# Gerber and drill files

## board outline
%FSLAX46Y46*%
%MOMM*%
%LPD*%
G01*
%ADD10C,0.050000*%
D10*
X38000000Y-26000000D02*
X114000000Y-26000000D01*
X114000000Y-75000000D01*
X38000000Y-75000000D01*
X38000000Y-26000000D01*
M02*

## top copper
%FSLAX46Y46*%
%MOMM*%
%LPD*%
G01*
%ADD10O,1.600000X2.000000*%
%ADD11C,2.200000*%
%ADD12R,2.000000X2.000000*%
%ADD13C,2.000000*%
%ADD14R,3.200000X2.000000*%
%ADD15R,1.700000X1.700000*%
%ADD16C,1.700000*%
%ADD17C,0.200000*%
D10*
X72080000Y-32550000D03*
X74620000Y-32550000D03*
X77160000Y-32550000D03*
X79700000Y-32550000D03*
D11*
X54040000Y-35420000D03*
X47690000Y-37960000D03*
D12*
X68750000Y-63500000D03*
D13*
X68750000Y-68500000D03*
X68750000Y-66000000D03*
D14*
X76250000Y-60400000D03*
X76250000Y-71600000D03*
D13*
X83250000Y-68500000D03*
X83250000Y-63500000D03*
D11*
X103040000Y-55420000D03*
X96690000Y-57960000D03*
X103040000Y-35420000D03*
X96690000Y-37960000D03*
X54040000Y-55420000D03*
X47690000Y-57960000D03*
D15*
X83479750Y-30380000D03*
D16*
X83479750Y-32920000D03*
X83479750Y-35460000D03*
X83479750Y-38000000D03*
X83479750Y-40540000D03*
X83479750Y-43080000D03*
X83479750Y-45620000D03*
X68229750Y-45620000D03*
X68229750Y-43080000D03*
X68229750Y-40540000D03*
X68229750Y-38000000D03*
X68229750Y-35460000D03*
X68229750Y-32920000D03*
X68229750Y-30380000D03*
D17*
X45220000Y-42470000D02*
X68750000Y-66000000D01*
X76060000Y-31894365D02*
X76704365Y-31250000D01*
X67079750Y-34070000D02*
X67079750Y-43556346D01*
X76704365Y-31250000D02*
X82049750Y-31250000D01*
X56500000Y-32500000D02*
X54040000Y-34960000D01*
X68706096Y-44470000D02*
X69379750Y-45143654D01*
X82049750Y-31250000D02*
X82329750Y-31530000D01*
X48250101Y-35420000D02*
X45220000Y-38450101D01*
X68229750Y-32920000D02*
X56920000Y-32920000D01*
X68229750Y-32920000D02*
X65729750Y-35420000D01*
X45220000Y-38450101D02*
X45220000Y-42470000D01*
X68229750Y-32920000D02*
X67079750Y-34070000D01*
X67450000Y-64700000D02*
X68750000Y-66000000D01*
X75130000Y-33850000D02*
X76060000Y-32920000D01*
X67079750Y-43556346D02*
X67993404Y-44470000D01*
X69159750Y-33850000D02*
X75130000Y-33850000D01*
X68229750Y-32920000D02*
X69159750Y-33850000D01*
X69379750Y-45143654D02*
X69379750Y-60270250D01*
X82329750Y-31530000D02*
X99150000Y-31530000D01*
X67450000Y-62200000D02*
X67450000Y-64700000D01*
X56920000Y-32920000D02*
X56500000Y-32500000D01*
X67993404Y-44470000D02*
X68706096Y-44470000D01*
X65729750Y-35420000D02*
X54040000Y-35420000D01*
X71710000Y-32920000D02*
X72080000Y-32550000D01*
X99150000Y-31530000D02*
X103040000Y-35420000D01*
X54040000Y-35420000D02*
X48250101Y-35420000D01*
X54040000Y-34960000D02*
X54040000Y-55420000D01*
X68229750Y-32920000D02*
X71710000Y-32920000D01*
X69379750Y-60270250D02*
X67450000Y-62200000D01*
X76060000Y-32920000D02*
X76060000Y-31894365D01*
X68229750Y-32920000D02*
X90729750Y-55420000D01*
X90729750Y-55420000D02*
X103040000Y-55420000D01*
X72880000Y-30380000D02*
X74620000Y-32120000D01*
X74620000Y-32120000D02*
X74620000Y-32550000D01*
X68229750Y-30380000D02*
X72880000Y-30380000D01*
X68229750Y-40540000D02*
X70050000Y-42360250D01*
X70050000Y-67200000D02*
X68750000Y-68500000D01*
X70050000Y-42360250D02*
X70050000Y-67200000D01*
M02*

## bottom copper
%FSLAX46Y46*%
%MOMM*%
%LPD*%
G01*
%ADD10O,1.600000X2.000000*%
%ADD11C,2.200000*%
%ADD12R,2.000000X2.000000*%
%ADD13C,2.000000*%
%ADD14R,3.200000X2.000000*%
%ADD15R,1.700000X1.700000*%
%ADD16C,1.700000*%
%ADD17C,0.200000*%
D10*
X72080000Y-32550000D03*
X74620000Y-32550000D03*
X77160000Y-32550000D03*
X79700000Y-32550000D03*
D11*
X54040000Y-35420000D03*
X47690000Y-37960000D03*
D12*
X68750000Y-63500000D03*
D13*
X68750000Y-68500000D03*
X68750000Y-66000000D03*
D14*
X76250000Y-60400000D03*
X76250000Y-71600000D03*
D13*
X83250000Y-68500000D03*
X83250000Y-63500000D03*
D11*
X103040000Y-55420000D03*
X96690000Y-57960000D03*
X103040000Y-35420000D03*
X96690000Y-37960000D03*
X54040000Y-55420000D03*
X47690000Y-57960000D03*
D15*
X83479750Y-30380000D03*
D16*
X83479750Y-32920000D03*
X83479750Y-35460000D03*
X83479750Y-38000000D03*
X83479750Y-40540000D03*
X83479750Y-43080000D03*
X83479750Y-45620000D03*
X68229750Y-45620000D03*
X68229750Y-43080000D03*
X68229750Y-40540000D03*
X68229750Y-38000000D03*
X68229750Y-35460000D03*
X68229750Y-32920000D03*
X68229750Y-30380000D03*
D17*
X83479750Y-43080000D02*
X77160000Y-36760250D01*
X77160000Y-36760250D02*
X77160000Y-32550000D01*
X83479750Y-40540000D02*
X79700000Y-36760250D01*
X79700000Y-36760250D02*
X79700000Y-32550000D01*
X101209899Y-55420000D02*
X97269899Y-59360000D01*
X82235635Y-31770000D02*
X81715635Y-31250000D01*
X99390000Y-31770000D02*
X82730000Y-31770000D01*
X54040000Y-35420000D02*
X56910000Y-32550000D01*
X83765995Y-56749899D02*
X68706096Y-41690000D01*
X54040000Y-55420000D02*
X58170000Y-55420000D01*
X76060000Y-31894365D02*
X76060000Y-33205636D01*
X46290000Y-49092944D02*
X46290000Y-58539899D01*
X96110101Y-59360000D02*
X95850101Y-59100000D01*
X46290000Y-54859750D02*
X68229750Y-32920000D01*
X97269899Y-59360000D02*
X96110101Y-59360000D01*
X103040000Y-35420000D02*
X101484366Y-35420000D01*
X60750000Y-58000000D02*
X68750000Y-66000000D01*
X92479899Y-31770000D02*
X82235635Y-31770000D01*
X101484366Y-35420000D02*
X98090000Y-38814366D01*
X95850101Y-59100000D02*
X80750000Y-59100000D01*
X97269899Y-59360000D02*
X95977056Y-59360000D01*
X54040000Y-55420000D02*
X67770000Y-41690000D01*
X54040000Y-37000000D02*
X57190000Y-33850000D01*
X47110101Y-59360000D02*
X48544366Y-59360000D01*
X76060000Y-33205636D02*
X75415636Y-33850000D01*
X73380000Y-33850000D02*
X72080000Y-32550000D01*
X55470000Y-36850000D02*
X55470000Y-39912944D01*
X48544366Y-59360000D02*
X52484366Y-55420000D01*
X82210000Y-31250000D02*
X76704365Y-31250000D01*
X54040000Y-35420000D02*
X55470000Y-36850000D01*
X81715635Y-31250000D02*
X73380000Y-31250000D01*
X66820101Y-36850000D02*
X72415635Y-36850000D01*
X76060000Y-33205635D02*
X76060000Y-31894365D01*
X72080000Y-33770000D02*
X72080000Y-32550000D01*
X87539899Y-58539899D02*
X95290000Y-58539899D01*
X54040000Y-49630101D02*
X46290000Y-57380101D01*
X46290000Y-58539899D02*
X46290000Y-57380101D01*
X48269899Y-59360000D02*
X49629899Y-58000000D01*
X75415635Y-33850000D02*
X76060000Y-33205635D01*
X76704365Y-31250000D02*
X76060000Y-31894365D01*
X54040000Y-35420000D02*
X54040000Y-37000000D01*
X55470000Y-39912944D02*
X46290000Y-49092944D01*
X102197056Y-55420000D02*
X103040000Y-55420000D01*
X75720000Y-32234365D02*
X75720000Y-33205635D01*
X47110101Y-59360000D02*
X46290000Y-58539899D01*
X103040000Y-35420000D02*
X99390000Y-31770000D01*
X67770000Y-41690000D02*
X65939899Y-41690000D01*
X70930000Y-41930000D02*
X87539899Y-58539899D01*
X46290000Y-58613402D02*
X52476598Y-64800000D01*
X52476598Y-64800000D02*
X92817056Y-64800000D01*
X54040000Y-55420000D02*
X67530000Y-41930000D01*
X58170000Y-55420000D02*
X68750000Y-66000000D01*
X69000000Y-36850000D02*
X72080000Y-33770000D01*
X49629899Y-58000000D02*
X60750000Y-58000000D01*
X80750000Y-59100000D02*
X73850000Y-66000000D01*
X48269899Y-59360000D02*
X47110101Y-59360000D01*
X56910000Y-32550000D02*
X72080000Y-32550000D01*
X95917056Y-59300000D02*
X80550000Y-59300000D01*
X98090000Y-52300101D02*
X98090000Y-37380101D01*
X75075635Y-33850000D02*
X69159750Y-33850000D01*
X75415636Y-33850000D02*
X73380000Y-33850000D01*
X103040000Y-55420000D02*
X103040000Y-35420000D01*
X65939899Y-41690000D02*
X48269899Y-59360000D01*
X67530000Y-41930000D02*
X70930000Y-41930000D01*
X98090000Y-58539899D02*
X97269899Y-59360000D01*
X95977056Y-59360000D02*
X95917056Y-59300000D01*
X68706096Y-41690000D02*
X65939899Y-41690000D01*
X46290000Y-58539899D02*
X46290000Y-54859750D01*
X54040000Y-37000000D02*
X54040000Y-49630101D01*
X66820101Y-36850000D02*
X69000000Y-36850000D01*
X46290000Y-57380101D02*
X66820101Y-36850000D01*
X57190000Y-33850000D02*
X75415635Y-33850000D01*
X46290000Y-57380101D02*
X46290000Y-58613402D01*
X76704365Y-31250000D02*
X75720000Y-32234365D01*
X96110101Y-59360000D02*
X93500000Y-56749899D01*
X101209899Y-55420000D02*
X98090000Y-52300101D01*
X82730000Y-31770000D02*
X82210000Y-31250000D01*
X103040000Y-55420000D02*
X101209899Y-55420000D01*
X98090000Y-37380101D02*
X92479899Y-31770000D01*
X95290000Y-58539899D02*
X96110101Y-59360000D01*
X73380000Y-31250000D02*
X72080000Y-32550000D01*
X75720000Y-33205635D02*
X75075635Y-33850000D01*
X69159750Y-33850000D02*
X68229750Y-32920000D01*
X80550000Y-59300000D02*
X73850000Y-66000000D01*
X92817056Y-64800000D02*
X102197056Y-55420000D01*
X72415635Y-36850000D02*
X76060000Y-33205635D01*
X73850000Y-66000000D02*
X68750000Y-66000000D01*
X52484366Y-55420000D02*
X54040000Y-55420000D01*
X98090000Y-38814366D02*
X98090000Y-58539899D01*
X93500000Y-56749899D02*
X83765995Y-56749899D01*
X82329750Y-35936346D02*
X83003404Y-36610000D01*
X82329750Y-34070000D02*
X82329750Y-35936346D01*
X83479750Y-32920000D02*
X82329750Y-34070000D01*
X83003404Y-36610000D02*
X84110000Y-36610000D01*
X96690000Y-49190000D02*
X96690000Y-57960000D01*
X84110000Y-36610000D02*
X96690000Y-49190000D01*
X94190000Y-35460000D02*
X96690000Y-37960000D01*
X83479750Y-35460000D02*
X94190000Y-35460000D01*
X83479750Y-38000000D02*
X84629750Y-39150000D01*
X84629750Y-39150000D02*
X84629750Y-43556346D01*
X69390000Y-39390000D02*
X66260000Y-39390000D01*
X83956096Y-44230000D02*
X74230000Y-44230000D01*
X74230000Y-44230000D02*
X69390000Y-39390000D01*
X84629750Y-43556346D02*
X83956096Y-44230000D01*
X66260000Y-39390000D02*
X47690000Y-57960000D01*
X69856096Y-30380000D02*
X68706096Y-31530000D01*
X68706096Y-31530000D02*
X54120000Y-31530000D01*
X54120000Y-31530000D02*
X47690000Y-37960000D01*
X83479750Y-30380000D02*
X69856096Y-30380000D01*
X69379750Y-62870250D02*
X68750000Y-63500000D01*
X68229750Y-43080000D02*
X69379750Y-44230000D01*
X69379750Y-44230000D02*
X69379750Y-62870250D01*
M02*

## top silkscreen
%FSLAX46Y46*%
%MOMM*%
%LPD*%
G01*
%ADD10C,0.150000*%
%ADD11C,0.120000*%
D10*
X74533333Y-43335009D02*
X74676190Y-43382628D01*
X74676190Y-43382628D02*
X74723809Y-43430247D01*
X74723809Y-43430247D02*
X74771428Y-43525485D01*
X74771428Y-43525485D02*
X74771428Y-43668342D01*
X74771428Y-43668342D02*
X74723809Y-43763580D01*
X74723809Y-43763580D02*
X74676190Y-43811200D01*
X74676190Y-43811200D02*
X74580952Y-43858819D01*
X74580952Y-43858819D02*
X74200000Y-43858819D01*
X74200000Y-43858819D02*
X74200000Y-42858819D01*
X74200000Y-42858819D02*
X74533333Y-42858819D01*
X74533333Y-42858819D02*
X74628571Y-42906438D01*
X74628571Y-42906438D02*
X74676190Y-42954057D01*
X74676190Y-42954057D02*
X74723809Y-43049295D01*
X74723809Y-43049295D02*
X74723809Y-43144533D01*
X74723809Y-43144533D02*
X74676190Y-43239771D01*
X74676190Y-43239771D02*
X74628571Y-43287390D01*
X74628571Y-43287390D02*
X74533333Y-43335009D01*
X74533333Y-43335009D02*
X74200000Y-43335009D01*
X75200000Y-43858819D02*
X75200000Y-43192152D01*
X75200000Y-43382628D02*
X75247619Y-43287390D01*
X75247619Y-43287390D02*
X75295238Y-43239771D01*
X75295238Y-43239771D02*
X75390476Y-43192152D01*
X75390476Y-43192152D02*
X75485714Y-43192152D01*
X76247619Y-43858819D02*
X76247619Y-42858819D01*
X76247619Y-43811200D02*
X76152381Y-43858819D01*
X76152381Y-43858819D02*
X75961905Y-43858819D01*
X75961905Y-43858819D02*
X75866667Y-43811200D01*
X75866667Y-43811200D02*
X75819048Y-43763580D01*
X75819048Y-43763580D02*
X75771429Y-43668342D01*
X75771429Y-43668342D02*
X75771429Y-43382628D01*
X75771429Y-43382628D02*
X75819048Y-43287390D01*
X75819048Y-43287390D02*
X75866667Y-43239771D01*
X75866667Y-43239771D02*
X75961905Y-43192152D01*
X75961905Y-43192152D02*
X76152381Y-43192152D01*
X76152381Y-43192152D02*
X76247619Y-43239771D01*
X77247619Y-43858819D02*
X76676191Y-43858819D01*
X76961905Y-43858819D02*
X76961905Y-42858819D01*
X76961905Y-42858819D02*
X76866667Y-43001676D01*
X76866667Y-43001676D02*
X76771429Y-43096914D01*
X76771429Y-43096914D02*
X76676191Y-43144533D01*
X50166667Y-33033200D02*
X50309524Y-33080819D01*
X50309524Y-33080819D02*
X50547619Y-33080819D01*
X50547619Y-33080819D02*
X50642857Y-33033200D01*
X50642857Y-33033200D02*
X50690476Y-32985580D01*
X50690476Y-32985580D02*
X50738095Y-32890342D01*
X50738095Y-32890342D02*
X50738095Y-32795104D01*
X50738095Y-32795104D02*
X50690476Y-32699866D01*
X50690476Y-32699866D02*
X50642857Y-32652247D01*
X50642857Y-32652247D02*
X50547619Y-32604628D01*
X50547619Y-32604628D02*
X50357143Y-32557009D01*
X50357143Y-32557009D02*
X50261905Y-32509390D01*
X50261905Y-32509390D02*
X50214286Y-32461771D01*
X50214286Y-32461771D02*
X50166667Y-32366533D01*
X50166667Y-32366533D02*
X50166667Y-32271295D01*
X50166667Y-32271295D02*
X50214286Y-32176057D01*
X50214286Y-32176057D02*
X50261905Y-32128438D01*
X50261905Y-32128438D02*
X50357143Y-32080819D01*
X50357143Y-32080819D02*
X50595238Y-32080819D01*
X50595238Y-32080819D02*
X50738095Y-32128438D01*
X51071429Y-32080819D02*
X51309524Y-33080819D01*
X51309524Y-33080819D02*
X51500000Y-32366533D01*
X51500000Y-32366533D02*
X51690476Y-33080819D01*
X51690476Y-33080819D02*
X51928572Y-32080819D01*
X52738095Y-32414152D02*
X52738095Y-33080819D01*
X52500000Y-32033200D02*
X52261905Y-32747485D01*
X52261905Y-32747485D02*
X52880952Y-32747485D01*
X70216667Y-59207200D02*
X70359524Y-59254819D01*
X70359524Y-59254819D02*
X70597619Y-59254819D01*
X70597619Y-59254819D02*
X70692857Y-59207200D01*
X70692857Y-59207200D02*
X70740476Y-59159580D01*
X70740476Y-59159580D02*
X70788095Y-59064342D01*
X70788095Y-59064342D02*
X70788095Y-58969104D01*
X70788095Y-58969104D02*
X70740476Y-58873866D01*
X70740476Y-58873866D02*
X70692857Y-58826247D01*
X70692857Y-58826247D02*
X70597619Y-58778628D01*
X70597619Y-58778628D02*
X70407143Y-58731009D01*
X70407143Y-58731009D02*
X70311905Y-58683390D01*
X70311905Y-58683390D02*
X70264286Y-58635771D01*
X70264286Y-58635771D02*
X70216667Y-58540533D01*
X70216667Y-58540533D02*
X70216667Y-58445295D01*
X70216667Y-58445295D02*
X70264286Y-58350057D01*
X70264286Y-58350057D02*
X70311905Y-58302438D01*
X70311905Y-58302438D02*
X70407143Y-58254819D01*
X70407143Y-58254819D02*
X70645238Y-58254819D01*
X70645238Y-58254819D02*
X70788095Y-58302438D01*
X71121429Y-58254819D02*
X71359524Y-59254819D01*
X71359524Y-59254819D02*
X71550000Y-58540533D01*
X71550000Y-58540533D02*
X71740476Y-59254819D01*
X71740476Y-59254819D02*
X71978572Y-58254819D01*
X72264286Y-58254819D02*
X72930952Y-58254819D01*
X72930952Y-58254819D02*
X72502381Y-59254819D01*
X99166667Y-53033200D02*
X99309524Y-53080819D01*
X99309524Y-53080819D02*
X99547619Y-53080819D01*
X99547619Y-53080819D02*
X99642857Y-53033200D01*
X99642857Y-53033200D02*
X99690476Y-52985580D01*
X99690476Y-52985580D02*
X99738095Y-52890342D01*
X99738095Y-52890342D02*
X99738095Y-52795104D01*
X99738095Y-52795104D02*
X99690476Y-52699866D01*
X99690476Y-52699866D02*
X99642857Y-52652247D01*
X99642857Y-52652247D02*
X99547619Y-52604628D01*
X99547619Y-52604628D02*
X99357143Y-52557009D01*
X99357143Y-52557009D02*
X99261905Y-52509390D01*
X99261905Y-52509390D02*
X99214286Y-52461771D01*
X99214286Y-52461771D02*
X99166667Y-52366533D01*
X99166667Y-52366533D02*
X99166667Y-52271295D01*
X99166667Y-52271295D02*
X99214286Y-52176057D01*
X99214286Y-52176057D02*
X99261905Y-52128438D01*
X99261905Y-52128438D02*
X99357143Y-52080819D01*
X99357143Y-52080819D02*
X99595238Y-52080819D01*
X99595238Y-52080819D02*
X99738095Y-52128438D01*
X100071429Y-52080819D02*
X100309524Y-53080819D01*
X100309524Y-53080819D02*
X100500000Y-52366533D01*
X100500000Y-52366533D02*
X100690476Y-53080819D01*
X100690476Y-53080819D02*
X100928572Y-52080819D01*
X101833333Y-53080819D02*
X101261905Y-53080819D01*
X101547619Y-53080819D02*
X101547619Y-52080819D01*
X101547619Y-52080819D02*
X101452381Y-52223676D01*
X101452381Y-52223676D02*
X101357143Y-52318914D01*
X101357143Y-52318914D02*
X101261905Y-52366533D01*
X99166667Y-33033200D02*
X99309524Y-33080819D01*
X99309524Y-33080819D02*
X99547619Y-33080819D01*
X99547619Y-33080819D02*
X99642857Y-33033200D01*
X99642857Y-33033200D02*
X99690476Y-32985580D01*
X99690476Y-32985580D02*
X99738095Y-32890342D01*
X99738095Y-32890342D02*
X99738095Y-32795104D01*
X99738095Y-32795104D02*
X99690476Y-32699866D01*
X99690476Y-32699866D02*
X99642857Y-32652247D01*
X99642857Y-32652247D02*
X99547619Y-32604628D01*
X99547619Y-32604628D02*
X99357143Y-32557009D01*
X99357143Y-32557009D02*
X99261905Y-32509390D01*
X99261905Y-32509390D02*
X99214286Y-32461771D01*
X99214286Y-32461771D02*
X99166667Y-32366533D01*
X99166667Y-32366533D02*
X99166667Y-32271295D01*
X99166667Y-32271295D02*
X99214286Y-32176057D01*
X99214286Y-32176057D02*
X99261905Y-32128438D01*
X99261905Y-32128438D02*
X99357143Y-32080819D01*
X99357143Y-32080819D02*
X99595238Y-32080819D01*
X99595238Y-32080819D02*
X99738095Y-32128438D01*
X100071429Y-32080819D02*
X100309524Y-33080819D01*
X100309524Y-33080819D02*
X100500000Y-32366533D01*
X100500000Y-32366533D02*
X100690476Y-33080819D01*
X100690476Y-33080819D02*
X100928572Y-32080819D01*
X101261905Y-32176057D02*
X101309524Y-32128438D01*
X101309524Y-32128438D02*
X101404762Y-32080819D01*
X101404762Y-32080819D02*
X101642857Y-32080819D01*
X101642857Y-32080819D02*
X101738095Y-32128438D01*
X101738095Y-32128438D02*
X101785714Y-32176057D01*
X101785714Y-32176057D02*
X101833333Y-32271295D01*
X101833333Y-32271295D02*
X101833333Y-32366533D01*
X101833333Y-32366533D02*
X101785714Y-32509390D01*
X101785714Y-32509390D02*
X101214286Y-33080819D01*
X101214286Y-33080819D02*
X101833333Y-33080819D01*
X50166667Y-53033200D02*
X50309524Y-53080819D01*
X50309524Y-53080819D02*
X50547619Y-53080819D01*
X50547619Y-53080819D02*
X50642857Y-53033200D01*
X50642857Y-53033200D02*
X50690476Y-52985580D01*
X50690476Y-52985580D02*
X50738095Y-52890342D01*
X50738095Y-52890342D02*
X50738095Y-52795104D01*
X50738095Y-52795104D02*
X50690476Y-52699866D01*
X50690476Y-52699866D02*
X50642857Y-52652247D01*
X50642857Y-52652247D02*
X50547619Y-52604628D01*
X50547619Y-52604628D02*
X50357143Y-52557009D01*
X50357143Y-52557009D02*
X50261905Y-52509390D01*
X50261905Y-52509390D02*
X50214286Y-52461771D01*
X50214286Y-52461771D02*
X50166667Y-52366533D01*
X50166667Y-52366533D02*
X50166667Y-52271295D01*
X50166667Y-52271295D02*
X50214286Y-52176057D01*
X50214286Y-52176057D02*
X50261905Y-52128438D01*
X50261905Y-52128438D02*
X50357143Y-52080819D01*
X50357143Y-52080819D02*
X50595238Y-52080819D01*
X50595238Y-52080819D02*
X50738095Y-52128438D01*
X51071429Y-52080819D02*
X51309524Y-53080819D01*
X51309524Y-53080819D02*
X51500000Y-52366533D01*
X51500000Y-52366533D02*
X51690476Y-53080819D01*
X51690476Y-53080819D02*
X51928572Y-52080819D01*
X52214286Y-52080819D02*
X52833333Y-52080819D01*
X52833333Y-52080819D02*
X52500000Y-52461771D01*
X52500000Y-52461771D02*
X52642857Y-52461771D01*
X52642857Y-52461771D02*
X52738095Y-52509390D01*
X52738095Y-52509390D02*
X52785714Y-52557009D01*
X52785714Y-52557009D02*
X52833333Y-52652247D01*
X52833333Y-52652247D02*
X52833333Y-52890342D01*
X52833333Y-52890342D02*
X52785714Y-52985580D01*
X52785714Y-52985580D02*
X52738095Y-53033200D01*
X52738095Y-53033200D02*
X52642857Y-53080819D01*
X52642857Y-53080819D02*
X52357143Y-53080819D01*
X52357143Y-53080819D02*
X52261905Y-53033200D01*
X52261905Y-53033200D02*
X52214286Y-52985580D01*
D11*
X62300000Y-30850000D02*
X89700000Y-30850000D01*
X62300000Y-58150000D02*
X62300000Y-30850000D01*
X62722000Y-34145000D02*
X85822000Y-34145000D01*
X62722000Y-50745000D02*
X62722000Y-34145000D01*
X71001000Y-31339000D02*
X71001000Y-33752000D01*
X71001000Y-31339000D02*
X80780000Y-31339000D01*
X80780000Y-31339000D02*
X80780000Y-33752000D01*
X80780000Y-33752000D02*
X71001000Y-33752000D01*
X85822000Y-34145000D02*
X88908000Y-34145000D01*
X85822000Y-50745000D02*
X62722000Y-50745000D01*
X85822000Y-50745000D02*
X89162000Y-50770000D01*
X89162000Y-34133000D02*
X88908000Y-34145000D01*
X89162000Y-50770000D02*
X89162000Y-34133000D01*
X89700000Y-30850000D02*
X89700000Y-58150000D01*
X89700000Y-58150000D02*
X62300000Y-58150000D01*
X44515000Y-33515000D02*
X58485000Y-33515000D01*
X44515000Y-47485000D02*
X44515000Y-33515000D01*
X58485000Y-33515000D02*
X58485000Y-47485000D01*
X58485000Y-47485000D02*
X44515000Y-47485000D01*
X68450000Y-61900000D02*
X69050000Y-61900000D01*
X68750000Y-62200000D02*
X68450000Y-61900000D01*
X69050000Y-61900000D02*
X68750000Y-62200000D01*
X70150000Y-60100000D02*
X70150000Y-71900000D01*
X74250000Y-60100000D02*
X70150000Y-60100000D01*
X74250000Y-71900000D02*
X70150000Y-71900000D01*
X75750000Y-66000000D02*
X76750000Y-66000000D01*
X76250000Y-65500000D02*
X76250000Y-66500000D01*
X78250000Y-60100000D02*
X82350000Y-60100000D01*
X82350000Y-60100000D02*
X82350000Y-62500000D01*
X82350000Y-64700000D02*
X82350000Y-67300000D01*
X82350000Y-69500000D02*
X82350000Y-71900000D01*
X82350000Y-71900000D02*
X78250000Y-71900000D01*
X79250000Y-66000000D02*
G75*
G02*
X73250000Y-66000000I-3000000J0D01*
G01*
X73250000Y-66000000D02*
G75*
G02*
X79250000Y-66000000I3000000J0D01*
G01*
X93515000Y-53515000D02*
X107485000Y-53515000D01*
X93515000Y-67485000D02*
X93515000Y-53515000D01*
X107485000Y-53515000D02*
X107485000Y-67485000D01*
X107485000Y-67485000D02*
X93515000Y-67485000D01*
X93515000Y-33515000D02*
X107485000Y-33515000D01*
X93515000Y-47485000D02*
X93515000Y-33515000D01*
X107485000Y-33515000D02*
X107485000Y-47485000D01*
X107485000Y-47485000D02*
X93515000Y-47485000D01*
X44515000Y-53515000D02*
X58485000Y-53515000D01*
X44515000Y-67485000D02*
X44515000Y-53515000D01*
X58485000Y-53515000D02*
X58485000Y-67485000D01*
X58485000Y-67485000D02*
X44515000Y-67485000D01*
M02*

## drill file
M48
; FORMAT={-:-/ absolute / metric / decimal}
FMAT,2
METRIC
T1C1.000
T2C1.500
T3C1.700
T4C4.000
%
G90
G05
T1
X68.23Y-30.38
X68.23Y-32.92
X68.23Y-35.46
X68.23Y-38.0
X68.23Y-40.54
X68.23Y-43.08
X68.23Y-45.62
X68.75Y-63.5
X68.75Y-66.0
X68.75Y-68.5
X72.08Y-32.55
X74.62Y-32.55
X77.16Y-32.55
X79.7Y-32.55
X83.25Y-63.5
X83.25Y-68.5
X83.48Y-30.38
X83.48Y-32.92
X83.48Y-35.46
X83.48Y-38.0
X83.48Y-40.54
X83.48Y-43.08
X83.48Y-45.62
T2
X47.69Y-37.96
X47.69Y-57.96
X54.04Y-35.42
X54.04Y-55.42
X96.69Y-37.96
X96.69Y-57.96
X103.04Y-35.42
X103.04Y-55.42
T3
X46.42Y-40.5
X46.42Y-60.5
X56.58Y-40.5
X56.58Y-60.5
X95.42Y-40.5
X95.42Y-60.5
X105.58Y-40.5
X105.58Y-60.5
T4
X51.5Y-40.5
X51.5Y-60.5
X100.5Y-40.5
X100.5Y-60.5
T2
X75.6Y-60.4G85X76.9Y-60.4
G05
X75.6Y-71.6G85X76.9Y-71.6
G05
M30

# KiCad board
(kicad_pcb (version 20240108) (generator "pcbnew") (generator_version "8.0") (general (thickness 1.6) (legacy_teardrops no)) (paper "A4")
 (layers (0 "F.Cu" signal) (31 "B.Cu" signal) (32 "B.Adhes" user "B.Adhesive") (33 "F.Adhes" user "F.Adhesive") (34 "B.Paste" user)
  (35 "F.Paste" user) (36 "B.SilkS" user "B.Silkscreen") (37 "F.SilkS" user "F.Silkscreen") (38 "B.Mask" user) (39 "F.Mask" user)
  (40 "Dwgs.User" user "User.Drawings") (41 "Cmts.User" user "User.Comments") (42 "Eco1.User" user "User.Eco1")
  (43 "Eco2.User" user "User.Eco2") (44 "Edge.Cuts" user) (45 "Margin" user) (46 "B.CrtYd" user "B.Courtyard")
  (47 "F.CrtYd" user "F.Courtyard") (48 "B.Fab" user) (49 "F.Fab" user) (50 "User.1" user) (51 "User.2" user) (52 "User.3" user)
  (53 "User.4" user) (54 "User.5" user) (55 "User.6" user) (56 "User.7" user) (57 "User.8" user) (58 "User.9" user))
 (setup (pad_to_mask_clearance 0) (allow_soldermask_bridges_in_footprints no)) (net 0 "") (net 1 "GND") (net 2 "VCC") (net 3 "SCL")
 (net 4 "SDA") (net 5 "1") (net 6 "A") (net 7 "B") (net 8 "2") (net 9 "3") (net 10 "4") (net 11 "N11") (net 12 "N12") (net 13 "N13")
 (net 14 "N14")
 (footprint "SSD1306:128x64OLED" (layer "F.Cu") (at 75.7 43.15)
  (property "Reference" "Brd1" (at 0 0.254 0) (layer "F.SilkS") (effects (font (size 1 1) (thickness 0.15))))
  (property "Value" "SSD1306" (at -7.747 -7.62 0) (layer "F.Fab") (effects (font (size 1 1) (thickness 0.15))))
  (fp_line (start -13.4 -12.3) (end 14 -12.3) (stroke (width 0.12) (type solid)) (layer "F.SilkS"))
  (fp_line (start -13.4 15) (end -13.4 -12.3) (stroke (width 0.12) (type solid)) (layer "F.SilkS"))
  (fp_line (start -12.978 -9.005) (end 10.122 -9.005) (stroke (width 0.12) (type solid)) (layer "F.SilkS"))
  (fp_line (start -12.978 7.595) (end -12.978 -9.005) (stroke (width 0.12) (type solid)) (layer "F.SilkS"))
  (fp_line (start -4.699 -11.811) (end -4.699 -9.398) (stroke (width 0.12) (type solid)) (layer "F.SilkS"))
  (fp_line (start -4.699 -11.811) (end 5.08 -11.811) (stroke (width 0.12) (type solid)) (layer "F.SilkS"))
  (fp_line (start 5.08 -11.811) (end 5.08 -9.398) (stroke (width 0.12) (type solid)) (layer "F.SilkS"))
  (fp_line (start 5.08 -9.398) (end -4.699 -9.398) (stroke (width 0.12) (type solid)) (layer "F.SilkS"))
  (fp_line (start 10.122 -9.005) (end 13.208 -9.005) (stroke (width 0.12) (type solid)) (layer "F.SilkS"))
  (fp_line (start 10.122 7.595) (end -12.978 7.595) (stroke (width 0.12) (type solid)) (layer "F.SilkS"))
  (fp_line (start 10.122 7.595) (end 13.462 7.62) (stroke (width 0.12) (type solid)) (layer "F.SilkS"))
  (fp_line (start 13.462 -9.017) (end 13.208 -9.005) (stroke (width 0.12) (type solid)) (layer "F.SilkS"))
  (fp_line (start 13.462 7.62) (end 13.462 -9.017) (stroke (width 0.12) (type solid)) (layer "F.SilkS"))
  (fp_line (start 14 -12.3) (end 14 15) (stroke (width 0.12) (type solid)) (layer "F.SilkS"))
  (fp_line (start 14 15) (end -13.4 15) (stroke (width 0.12) (type solid)) (layer "F.SilkS"))
  (pad "1" thru_hole oval (at -3.62 -10.6 90) (size 2 1.6) (drill 1) (layers "*.Cu" "*.Mask") (remove_unused_layers no) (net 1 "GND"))
  (pad "2" thru_hole oval (at -1.08 -10.6 90) (size 2 1.6) (drill 1) (layers "*.Cu" "*.Mask") (remove_unused_layers no) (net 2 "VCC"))
  (pad "3" thru_hole oval (at 1.46 -10.6 90) (size 2 1.6) (drill 1) (layers "*.Cu" "*.Mask") (remove_unused_layers no) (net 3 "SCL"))
  (pad "4" thru_hole oval (at 4 -10.6 90) (size 2 1.6) (drill 1) (layers "*.Cu" "*.Mask") (remove_unused_layers no) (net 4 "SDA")))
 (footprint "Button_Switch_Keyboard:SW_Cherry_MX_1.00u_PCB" (layer "F.Cu") (at 54.04 35.42)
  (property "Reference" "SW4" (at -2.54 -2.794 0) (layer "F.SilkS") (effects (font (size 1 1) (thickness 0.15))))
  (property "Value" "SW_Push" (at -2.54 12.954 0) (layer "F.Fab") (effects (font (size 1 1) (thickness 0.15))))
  (fp_line (start -9.525 -1.905) (end 4.445 -1.905) (stroke (width 0.12) (type solid)) (layer "F.SilkS"))
  (fp_line (start -9.525 12.065) (end -9.525 -1.905) (stroke (width 0.12) (type solid)) (layer "F.SilkS"))
  (fp_line (start 4.445 -1.905) (end 4.445 12.065) (stroke (width 0.12) (type solid)) (layer "F.SilkS"))
  (fp_line (start 4.445 12.065) (end -9.525 12.065) (stroke (width 0.12) (type solid)) (layer "F.SilkS"))
  (pad "" np_thru_hole circle (at -7.62 5.08) (size 1.7 1.7) (drill 1.7) (layers "*.Cu" "*.Mask"))
  (pad "" np_thru_hole circle (at -2.54 5.08) (size 4 4) (drill 4) (layers "*.Cu" "*.Mask"))
  (pad "" np_thru_hole circle (at 2.54 5.08) (size 1.7 1.7) (drill 1.7) (layers "*.Cu" "*.Mask"))
  (pad "1" thru_hole circle (at 0 0) (size 2.2 2.2) (drill 1.5) (layers "*.Cu" "*.Mask") (remove_unused_layers no) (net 1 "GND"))
  (pad "2" thru_hole circle (at -6.35 2.54) (size 2.2 2.2) (drill 1.5) (layers "*.Cu" "*.Mask") (remove_unused_layers no) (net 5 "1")))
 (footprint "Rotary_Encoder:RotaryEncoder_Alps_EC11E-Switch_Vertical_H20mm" (layer "F.Cu") (at 68.75 63.5)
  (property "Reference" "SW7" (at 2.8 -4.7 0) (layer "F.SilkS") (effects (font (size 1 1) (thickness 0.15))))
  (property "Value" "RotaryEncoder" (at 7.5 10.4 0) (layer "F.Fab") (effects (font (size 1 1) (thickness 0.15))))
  (fp_line (start -0.3 -1.6) (end 0.3 -1.6) (stroke (width 0.12) (type solid)) (layer "F.SilkS"))
  (fp_line (start 0 -1.3) (end -0.3 -1.6) (stroke (width 0.12) (type solid)) (layer "F.SilkS"))
  (fp_line (start 0.3 -1.6) (end 0 -1.3) (stroke (width 0.12) (type solid)) (layer "F.SilkS"))
  (fp_line (start 1.4 -3.4) (end 1.4 8.4) (stroke (width 0.12) (type solid)) (layer "F.SilkS"))
  (fp_line (start 5.5 -3.4) (end 1.4 -3.4) (stroke (width 0.12) (type solid)) (layer "F.SilkS"))
  (fp_line (start 5.5 8.4) (end 1.4 8.4) (stroke (width 0.12) (type solid)) (layer "F.SilkS"))
  (fp_line (start 7 2.5) (end 8 2.5) (stroke (width 0.12) (type solid)) (layer "F.SilkS"))
  (fp_line (start 7.5 2) (end 7.5 3) (stroke (width 0.12) (type solid)) (layer "F.SilkS"))
  (fp_line (start 9.5 -3.4) (end 13.6 -3.4) (stroke (width 0.12) (type solid)) (layer "F.SilkS"))
  (fp_line (start 13.6 -3.4) (end 13.6 -1) (stroke (width 0.12) (type solid)) (layer "F.SilkS"))
  (fp_line (start 13.6 1.2) (end 13.6 3.8) (stroke (width 0.12) (type solid)) (layer "F.SilkS"))
  (fp_line (start 13.6 6) (end 13.6 8.4) (stroke (width 0.12) (type solid)) (layer "F.SilkS"))
  (fp_line (start 13.6 8.4) (end 9.5 8.4) (stroke (width 0.12) (type solid)) (layer "F.SilkS"))
  (fp_circle (center 7.5 2.5) (end 10.5 2.5) (stroke (width 0.12) (type solid)) (fill none) (layer "F.SilkS"))
  (pad "A" thru_hole rect (at 0 0) (size 2 2) (drill 1) (layers "*.Cu" "*.Mask") (remove_unused_layers no) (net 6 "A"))
  (pad "B" thru_hole circle (at 0 5) (size 2 2) (drill 1) (layers "*.Cu" "*.Mask") (remove_unused_layers no) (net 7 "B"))
  (pad "C" thru_hole circle (at 0 2.5) (size 2 2) (drill 1) (layers "*.Cu" "*.Mask") (remove_unused_layers no) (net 1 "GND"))
  (pad "MP" thru_hole rect (at 7.5 -3.1) (size 3.2 2) (drill oval 2.8 1.5) (layers "*.Cu" "*.Mask") (remove_unused_layers no))
  (pad "MP" thru_hole rect (at 7.5 8.1) (size 3.2 2) (drill oval 2.8 1.5) (layers "*.Cu" "*.Mask") (remove_unused_layers no))
  (pad "S1" thru_hole circle (at 14.5 5) (size 2 2) (drill 1) (layers "*.Cu" "*.Mask") (remove_unused_layers no))
  (pad "S2" thru_hole circle (at 14.5 0) (size 2 2) (drill 1) (layers "*.Cu" "*.Mask") (remove_unused_layers no)))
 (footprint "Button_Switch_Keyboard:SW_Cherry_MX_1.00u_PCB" (layer "F.Cu") (at 103.04 55.42)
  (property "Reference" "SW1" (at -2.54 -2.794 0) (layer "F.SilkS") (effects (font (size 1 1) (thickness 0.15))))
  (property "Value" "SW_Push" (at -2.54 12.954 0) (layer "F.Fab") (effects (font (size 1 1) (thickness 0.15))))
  (fp_line (start -9.525 -1.905) (end 4.445 -1.905) (stroke (width 0.12) (type solid)) (layer "F.SilkS"))
  (fp_line (start -9.525 12.065) (end -9.525 -1.905) (stroke (width 0.12) (type solid)) (layer "F.SilkS"))
  (fp_line (start 4.445 -1.905) (end 4.445 12.065) (stroke (width 0.12) (type solid)) (layer "F.SilkS"))
  (fp_line (start 4.445 12.065) (end -9.525 12.065) (stroke (width 0.12) (type solid)) (layer "F.SilkS"))
  (pad "" np_thru_hole circle (at -7.62 5.08) (size 1.7 1.7) (drill 1.7) (layers "*.Cu" "*.Mask"))
  (pad "" np_thru_hole circle (at -2.54 5.08) (size 4 4) (drill 4) (layers "*.Cu" "*.Mask"))
  (pad "" np_thru_hole circle (at 2.54 5.08) (size 1.7 1.7) (drill 1.7) (layers "*.Cu" "*.Mask"))
  (pad "1" thru_hole circle (at 0 0) (size 2.2 2.2) (drill 1.5) (layers "*.Cu" "*.Mask") (remove_unused_layers no) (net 1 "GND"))
  (pad "2" thru_hole circle (at -6.35 2.54) (size 2.2 2.2) (drill 1.5) (layers "*.Cu" "*.Mask") (remove_unused_layers no) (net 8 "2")))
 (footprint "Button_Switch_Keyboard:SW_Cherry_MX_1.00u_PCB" (layer "F.Cu") (at 103.04 35.42)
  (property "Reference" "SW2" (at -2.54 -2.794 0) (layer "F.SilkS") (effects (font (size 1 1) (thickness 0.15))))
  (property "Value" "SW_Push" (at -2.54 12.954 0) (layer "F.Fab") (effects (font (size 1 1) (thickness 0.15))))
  (fp_line (start -9.525 -1.905) (end 4.445 -1.905) (stroke (width 0.12) (type solid)) (layer "F.SilkS"))
  (fp_line (start -9.525 12.065) (end -9.525 -1.905) (stroke (width 0.12) (type solid)) (layer "F.SilkS"))
  (fp_line (start 4.445 -1.905) (end 4.445 12.065) (stroke (width 0.12) (type solid)) (layer "F.SilkS"))
  (fp_line (start 4.445 12.065) (end -9.525 12.065) (stroke (width 0.12) (type solid)) (layer "F.SilkS"))
  (pad "" np_thru_hole circle (at -7.62 5.08) (size 1.7 1.7) (drill 1.7) (layers "*.Cu" "*.Mask"))
  (pad "" np_thru_hole circle (at -2.54 5.08) (size 4 4) (drill 4) (layers "*.Cu" "*.Mask"))
  (pad "" np_thru_hole circle (at 2.54 5.08) (size 1.7 1.7) (drill 1.7) (layers "*.Cu" "*.Mask"))
  (pad "1" thru_hole circle (at 0 0) (size 2.2 2.2) (drill 1.5) (layers "*.Cu" "*.Mask") (remove_unused_layers no) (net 1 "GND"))
  (pad "2" thru_hole circle (at -6.35 2.54) (size 2.2 2.2) (drill 1.5) (layers "*.Cu" "*.Mask") (remove_unused_layers no) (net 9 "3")))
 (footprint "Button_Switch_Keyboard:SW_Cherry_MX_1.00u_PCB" (layer "F.Cu") (at 54.04 55.42)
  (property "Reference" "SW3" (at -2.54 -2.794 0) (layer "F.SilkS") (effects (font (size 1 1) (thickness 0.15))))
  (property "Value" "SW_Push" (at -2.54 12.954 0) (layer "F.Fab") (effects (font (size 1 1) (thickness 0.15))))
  (fp_line (start -9.525 -1.905) (end 4.445 -1.905) (stroke (width 0.12) (type solid)) (layer "F.SilkS"))
  (fp_line (start -9.525 12.065) (end -9.525 -1.905) (stroke (width 0.12) (type solid)) (layer "F.SilkS"))
  (fp_line (start 4.445 -1.905) (end 4.445 12.065) (stroke (width 0.12) (type solid)) (layer "F.SilkS"))
  (fp_line (start 4.445 12.065) (end -9.525 12.065) (stroke (width 0.12) (type solid)) (layer "F.SilkS"))
  (pad "" np_thru_hole circle (at -7.62 5.08) (size 1.7 1.7) (drill 1.7) (layers "*.Cu" "*.Mask"))
  (pad "" np_thru_hole circle (at -2.54 5.08) (size 4 4) (drill 4) (layers "*.Cu" "*.Mask"))
  (pad "" np_thru_hole circle (at 2.54 5.08) (size 1.7 1.7) (drill 1.7) (layers "*.Cu" "*.Mask"))
  (pad "1" thru_hole circle (at 0 0) (size 2.2 2.2) (drill 1.5) (layers "*.Cu" "*.Mask") (remove_unused_layers no) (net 1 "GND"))
  (pad "2" thru_hole circle (at -6.35 2.54) (size 2.2 2.2) (drill 1.5) (layers "*.Cu" "*.Mask") (remove_unused_layers no) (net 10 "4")))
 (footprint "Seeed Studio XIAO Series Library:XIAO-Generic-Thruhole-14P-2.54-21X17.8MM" (layer "B.Cu") (at 75.85475 38 180)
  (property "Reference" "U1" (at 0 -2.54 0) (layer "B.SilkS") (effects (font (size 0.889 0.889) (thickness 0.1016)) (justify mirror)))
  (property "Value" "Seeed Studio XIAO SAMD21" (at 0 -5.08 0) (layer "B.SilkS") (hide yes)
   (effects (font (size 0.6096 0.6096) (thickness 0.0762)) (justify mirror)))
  (pad "1" thru_hole rect (at -7.625 7.62 180) (size 1.7 1.7) (drill 1) (layers "*.Cu" "*.Mask") (remove_unused_layers no) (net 5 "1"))
  (pad "2" thru_hole circle (at -7.625 5.08 180) (size 1.7 1.7) (drill 1) (layers "*.Cu" "*.Mask") (remove_unused_layers no) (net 8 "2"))
  (pad "3" thru_hole circle (at -7.625 2.54 180) (size 1.7 1.7) (drill 1) (layers "*.Cu" "*.Mask") (remove_unused_layers no) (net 9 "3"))
  (pad "4" thru_hole circle (at -7.625 0 180) (size 1.7 1.7) (drill 1) (layers "*.Cu" "*.Mask") (remove_unused_layers no) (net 10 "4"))
  (pad "5" thru_hole circle (at -7.625 -2.54 180) (size 1.7 1.7) (drill 1) (layers "*.Cu" "*.Mask") (remove_unused_layers no) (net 4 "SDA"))
  (pad "6" thru_hole circle (at -7.625 -5.08) (size 1.7 1.7) (drill 1) (layers "*.Cu" "*.Mask") (remove_unused_layers no) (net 3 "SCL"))
  (pad "7" thru_hole circle (at -7.625 -7.62 180) (size 1.7 1.7) (drill 1) (layers "*.Cu" "*.Mask") (remove_unused_layers no) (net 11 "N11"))
  (pad "8" thru_hole circle (at 7.625 -7.62 180) (size 1.7 1.7) (drill 1) (layers "*.Cu" "*.Mask") (remove_unused_layers no) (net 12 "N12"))
  (pad "9" thru_hole circle (at 7.625 -5.08 180) (size 1.7 1.7) (drill 1) (layers "*.Cu" "*.Mask") (remove_unused_layers no) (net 6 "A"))
  (pad "10" thru_hole circle (at 7.625 -2.54 180) (size 1.7 1.7) (drill 1) (layers "*.Cu" "*.Mask") (remove_unused_layers no) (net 7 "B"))
  (pad "11" thru_hole circle (at 7.625 0 180) (size 1.7 1.7) (drill 1) (layers "*.Cu" "*.Mask") (remove_unused_layers no) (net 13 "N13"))
  (pad "12" thru_hole circle (at 7.625 2.54 180) (size 1.7 1.7) (drill 1) (layers "*.Cu" "*.Mask") (remove_unused_layers no) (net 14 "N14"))
  (pad "13" thru_hole circle (at 7.625 5.08 180) (size 1.7 1.7) (drill 1) (layers "*.Cu" "*.Mask") (remove_unused_layers no) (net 1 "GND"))
  (pad "14" thru_hole circle (at 7.625 7.62 180) (size 1.7 1.7) (drill 1) (layers "*.Cu" "*.Mask") (remove_unused_layers no) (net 2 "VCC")))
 (gr_rect (start 38 26) (end 114 75) (stroke (width 0.05) (type default)) (fill none) (layer "Edge.Cuts"))
 (segment (start 83.47975 43.08) (end 77.16 36.76025) (width 0.2) (layer "B.Cu") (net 3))
 (segment (start 77.16 36.76025) (end 77.16 32.55) (width 0.2) (layer "B.Cu") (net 3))
 (segment (start 83.47975 40.54) (end 79.7 36.76025) (width 0.2) (layer "B.Cu") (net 4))
 (segment (start 79.7 36.76025) (end 79.7 32.55) (width 0.2) (layer "B.Cu") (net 4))
 (segment (start 45.22 42.47) (end 68.75 66) (width 0.2) (layer "F.Cu") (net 1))
 (segment (start 76.06 31.894365) (end 76.704365 31.25) (width 0.2) (layer "F.Cu") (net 1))
 (segment (start 67.07975 34.07) (end 67.07975 43.556346) (width 0.2) (layer "F.Cu") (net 1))
 (segment (start 76.704365 31.25) (end 82.04975 31.25) (width 0.2) (layer "F.Cu") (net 1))
 (segment (start 56.5 32.5) (end 54.04 34.96) (width 0.2) (layer "F.Cu") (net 1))
 (segment (start 68.706096 44.47) (end 69.37975 45.143654) (width 0.2) (layer "F.Cu") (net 1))
 (segment (start 82.04975 31.25) (end 82.32975 31.53) (width 0.2) (layer "F.Cu") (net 1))
 (segment (start 48.250101 35.42) (end 45.22 38.450101) (width 0.2) (layer "F.Cu") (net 1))
 (segment (start 68.22975 32.92) (end 56.92 32.92) (width 0.2) (layer "F.Cu") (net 1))
 (segment (start 68.22975 32.92) (end 65.72975 35.42) (width 0.2) (layer "F.Cu") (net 1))
 (segment (start 45.22 38.450101) (end 45.22 42.47) (width 0.2) (layer "F.Cu") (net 1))
 (segment (start 68.22975 32.92) (end 67.07975 34.07) (width 0.2) (layer "F.Cu") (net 1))
 (segment (start 67.45 64.7) (end 68.75 66) (width 0.2) (layer "F.Cu") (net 1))
 (segment (start 75.13 33.85) (end 76.06 32.92) (width 0.2) (layer "F.Cu") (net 1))
 (segment (start 67.07975 43.556346) (end 67.993404 44.47) (width 0.2) (layer "F.Cu") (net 1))
 (segment (start 69.15975 33.85) (end 75.13 33.85) (width 0.2) (layer "F.Cu") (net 1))
 (segment (start 68.22975 32.92) (end 69.15975 33.85) (width 0.2) (layer "F.Cu") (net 1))
 (segment (start 69.37975 45.143654) (end 69.37975 60.27025) (width 0.2) (layer "F.Cu") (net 1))
 (segment (start 82.32975 31.53) (end 99.15 31.53) (width 0.2) (layer "F.Cu") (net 1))
 (segment (start 67.45 62.2) (end 67.45 64.7) (width 0.2) (layer "F.Cu") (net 1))
 (segment (start 56.92 32.92) (end 56.5 32.5) (width 0.2) (layer "F.Cu") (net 1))
 (segment (start 67.993404 44.47) (end 68.706096 44.47) (width 0.2) (layer "F.Cu") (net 1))
 (segment (start 65.72975 35.42) (end 54.04 35.42) (width 0.2) (layer "F.Cu") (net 1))
 (segment (start 71.71 32.92) (end 72.08 32.55) (width 0.2) (layer "F.Cu") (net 1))
 (segment (start 99.15 31.53) (end 103.04 35.42) (width 0.2) (layer "F.Cu") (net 1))
 (segment (start 54.04 35.42) (end 48.250101 35.42) (width 0.2) (layer "F.Cu") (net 1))
 (segment (start 54.04 34.96) (end 54.04 55.42) (width 0.2) (layer "F.Cu") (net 1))
 (segment (start 68.22975 32.92) (end 71.71 32.92) (width 0.2) (layer "F.Cu") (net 1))
 (segment (start 69.37975 60.27025) (end 67.45 62.2) (width 0.2) (layer "F.Cu") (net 1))
 (segment (start 76.06 32.92) (end 76.06 31.894365) (width 0.2) (layer "F.Cu") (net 1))
 (segment (start 68.22975 32.92) (end 90.72975 55.42) (width 0.2) (layer "F.Cu") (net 1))
 (segment (start 90.72975 55.42) (end 103.04 55.42) (width 0.2) (layer "F.Cu") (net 1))
 (segment (start 101.209899 55.42) (end 97.269899 59.36) (width 0.2) (layer "B.Cu") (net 1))
 (segment (start 82.235635 31.77) (end 81.715635 31.25) (width 0.2) (layer "B.Cu") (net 1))
 (segment (start 99.39 31.77) (end 82.73 31.77) (width 0.2) (layer "B.Cu") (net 1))
 (segment (start 54.04 35.42) (end 56.91 32.55) (width 0.2) (layer "B.Cu") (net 1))
 (segment (start 83.765995 56.749899) (end 68.706096 41.69) (width 0.2) (layer "B.Cu") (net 1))
 (segment (start 54.04 55.42) (end 58.17 55.42) (width 0.2) (layer "B.Cu") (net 1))
 (segment (start 76.06 31.894365) (end 76.06 33.205636) (width 0.2) (layer "B.Cu") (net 1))
 (segment (start 46.29 49.092944) (end 46.29 58.539899) (width 0.2) (layer "B.Cu") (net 1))
 (segment (start 96.110101 59.36) (end 95.850101 59.1) (width 0.2) (layer "B.Cu") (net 1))
 (segment (start 46.29 54.85975) (end 68.22975 32.92) (width 0.2) (layer "B.Cu") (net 1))
 (segment (start 97.269899 59.36) (end 96.110101 59.36) (width 0.2) (layer "B.Cu") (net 1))
 (segment (start 103.04 35.42) (end 101.484366 35.42) (width 0.2) (layer "B.Cu") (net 1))
 (segment (start 60.75 58) (end 68.75 66) (width 0.2) (layer "B.Cu") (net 1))
 (segment (start 92.479899 31.77) (end 82.235635 31.77) (width 0.2) (layer "B.Cu") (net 1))
 (segment (start 101.484366 35.42) (end 98.09 38.814366) (width 0.2) (layer "B.Cu") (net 1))
 (segment (start 95.850101 59.1) (end 80.75 59.1) (width 0.2) (layer "B.Cu") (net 1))
 (segment (start 97.269899 59.36) (end 95.977056 59.36) (width 0.2) (layer "B.Cu") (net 1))
 (segment (start 54.04 55.42) (end 67.77 41.69) (width 0.2) (layer "B.Cu") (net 1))
 (segment (start 54.04 37) (end 57.19 33.85) (width 0.2) (layer "B.Cu") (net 1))
 (segment (start 47.110101 59.36) (end 48.544366 59.36) (width 0.2) (layer "B.Cu") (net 1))
 (segment (start 76.06 33.205636) (end 75.415636 33.85) (width 0.2) (layer "B.Cu") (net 1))
 (segment (start 73.38 33.85) (end 72.08 32.55) (width 0.2) (layer "B.Cu") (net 1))
 (segment (start 55.47 36.85) (end 55.47 39.912944) (width 0.2) (layer "B.Cu") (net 1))
 (segment (start 48.544366 59.36) (end 52.484366 55.42) (width 0.2) (layer "B.Cu") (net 1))
 (segment (start 82.21 31.25) (end 76.704365 31.25) (width 0.2) (layer "B.Cu") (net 1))
 (segment (start 54.04 35.42) (end 55.47 36.85) (width 0.2) (layer "B.Cu") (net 1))
 (segment (start 81.715635 31.25) (end 73.38 31.25) (width 0.2) (layer "B.Cu") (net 1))
 (segment (start 66.820101 36.85) (end 72.415635 36.85) (width 0.2) (layer "B.Cu") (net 1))
 (segment (start 76.06 33.205635) (end 76.06 31.894365) (width 0.2) (layer "B.Cu") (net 1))
 (segment (start 72.08 33.77) (end 72.08 32.55) (width 0.2) (layer "B.Cu") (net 1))
 (segment (start 87.539899 58.539899) (end 95.29 58.539899) (width 0.2) (layer "B.Cu") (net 1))
 (segment (start 54.04 49.630101) (end 46.29 57.380101) (width 0.2) (layer "B.Cu") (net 1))
 (segment (start 46.29 58.539899) (end 46.29 57.380101) (width 0.2) (layer "B.Cu") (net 1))
 (segment (start 48.269899 59.36) (end 49.629899 58) (width 0.2) (layer "B.Cu") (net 1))
 (segment (start 75.415635 33.85) (end 76.06 33.205635) (width 0.2) (layer "B.Cu") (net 1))
 (segment (start 76.704365 31.25) (end 76.06 31.894365) (width 0.2) (layer "B.Cu") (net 1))
 (segment (start 54.04 35.42) (end 54.04 37) (width 0.2) (layer "B.Cu") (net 1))
 (segment (start 55.47 39.912944) (end 46.29 49.092944) (width 0.2) (layer "B.Cu") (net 1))
 (segment (start 102.197056 55.42) (end 103.04 55.42) (width 0.2) (layer "B.Cu") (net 1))
 (segment (start 75.72 32.234365) (end 75.72 33.205635) (width 0.2) (layer "B.Cu") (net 1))
 (segment (start 47.110101 59.36) (end 46.29 58.539899) (width 0.2) (layer "B.Cu") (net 1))
 (segment (start 103.04 35.42) (end 99.39 31.77) (width 0.2) (layer "B.Cu") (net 1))
 (segment (start 67.77 41.69) (end 65.939899 41.69) (width 0.2) (layer "B.Cu") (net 1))
 (segment (start 70.93 41.93) (end 87.539899 58.539899) (width 0.2) (layer "B.Cu") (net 1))
 (segment (start 46.29 58.613402) (end 52.476598 64.8) (width 0.2) (layer "B.Cu") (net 1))
 (segment (start 52.476598 64.8) (end 92.817056 64.8) (width 0.2) (layer "B.Cu") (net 1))
 (segment (start 54.04 55.42) (end 67.53 41.93) (width 0.2) (layer "B.Cu") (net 1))
 (segment (start 58.17 55.42) (end 68.75 66) (width 0.2) (layer "B.Cu") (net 1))
 (segment (start 69 36.85) (end 72.08 33.77) (width 0.2) (layer "B.Cu") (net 1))
 (segment (start 49.629899 58) (end 60.75 58) (width 0.2) (layer "B.Cu") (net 1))
 (segment (start 80.75 59.1) (end 73.85 66) (width 0.2) (layer "B.Cu") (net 1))
 (segment (start 48.269899 59.36) (end 47.110101 59.36) (width 0.2) (layer "B.Cu") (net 1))
 (segment (start 56.91 32.55) (end 72.08 32.55) (width 0.2) (layer "B.Cu") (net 1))
 (segment (start 95.917056 59.3) (end 80.55 59.3) (width 0.2) (layer "B.Cu") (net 1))
 (segment (start 98.09 52.300101) (end 98.09 37.380101) (width 0.2) (layer "B.Cu") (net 1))
 (segment (start 75.075635 33.85) (end 69.15975 33.85) (width 0.2) (layer "B.Cu") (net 1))
 (segment (start 75.415636 33.85) (end 73.38 33.85) (width 0.2) (layer "B.Cu") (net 1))
 (segment (start 103.04 55.42) (end 103.04 35.42) (width 0.2) (layer "B.Cu") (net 1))
 (segment (start 65.939899 41.69) (end 48.269899 59.36) (width 0.2) (layer "B.Cu") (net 1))
 (segment (start 67.53 41.93) (end 70.93 41.93) (width 0.2) (layer "B.Cu") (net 1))
 (segment (start 98.09 58.539899) (end 97.269899 59.36) (width 0.2) (layer "B.Cu") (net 1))
 (segment (start 95.977056 59.36) (end 95.917056 59.3) (width 0.2) (layer "B.Cu") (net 1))
 (segment (start 68.706096 41.69) (end 65.939899 41.69) (width 0.2) (layer "B.Cu") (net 1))
 (segment (start 46.29 58.539899) (end 46.29 54.85975) (width 0.2) (layer "B.Cu") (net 1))
 (segment (start 54.04 37) (end 54.04 49.630101) (width 0.2) (layer "B.Cu") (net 1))
 (segment (start 66.820101 36.85) (end 69 36.85) (width 0.2) (layer "B.Cu") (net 1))
 (segment (start 46.29 57.380101) (end 66.820101 36.85) (width 0.2) (layer "B.Cu") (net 1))
 (segment (start 57.19 33.85) (end 75.415635 33.85) (width 0.2) (layer "B.Cu") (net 1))
 (segment (start 46.29 57.380101) (end 46.29 58.613402) (width 0.2) (layer "B.Cu") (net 1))
 (segment (start 76.704365 31.25) (end 75.72 32.234365) (width 0.2) (layer "B.Cu") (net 1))
 (segment (start 96.110101 59.36) (end 93.5 56.749899) (width 0.2) (layer "B.Cu") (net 1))
 (segment (start 101.209899 55.42) (end 98.09 52.300101) (width 0.2) (layer "B.Cu") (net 1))
 (segment (start 82.73 31.77) (end 82.21 31.25) (width 0.2) (layer "B.Cu") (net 1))
 (segment (start 103.04 55.42) (end 101.209899 55.42) (width 0.2) (layer "B.Cu") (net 1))
 (segment (start 98.09 37.380101) (end 92.479899 31.77) (width 0.2) (layer "B.Cu") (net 1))
 (segment (start 95.29 58.539899) (end 96.110101 59.36) (width 0.2) (layer "B.Cu") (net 1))
 (segment (start 73.38 31.25) (end 72.08 32.55) (width 0.2) (layer "B.Cu") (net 1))
 (segment (start 75.72 33.205635) (end 75.075635 33.85) (width 0.2) (layer "B.Cu") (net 1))
 (segment (start 69.15975 33.85) (end 68.22975 32.92) (width 0.2) (layer "B.Cu") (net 1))
 (segment (start 80.55 59.3) (end 73.85 66) (width 0.2) (layer "B.Cu") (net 1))
 (segment (start 92.817056 64.8) (end 102.197056 55.42) (width 0.2) (layer "B.Cu") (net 1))
 (segment (start 72.415635 36.85) (end 76.06 33.205635) (width 0.2) (layer "B.Cu") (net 1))
 (segment (start 73.85 66) (end 68.75 66) (width 0.2) (layer "B.Cu") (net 1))
 (segment (start 52.484366 55.42) (end 54.04 55.42) (width 0.2) (layer "B.Cu") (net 1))
 (segment (start 98.09 38.814366) (end 98.09 58.539899) (width 0.2) (layer "B.Cu") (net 1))
 (segment (start 93.5 56.749899) (end 83.765995 56.749899) (width 0.2) (layer "B.Cu") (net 1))
 (segment (start 72.88 30.38) (end 74.62 32.12) (width 0.2) (layer "F.Cu") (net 2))
 (segment (start 74.62 32.12) (end 74.62 32.55) (width 0.2) (layer "F.Cu") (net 2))
 (segment (start 68.22975 30.38) (end 72.88 30.38) (width 0.2) (layer "F.Cu") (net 2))
 (segment (start 82.32975 35.936346) (end 83.003404 36.61) (width 0.2) (layer "B.Cu") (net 8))
 (segment (start 82.32975 34.07) (end 82.32975 35.936346) (width 0.2) (layer "B.Cu") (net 8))
 (segment (start 83.47975 32.92) (end 82.32975 34.07) (width 0.2) (layer "B.Cu") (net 8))
 (segment (start 83.003404 36.61) (end 84.11 36.61) (width 0.2) (layer "B.Cu") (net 8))
 (segment (start 96.69 49.19) (end 96.69 57.96) (width 0.2) (layer "B.Cu") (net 8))
 (segment (start 84.11 36.61) (end 96.69 49.19) (width 0.2) (layer "B.Cu") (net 8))
 (segment (start 94.19 35.46) (end 96.69 37.96) (width 0.2) (layer "B.Cu") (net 9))
 (segment (start 83.47975 35.46) (end 94.19 35.46) (width 0.2) (layer "B.Cu") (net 9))
 (segment (start 83.47975 38) (end 84.62975 39.15) (width 0.2) (layer "B.Cu") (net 10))
 (segment (start 84.62975 39.15) (end 84.62975 43.556346) (width 0.2) (layer "B.Cu") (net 10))
 (segment (start 69.39 39.39) (end 66.26 39.39) (width 0.2) (layer "B.Cu") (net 10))
 (segment (start 83.956096 44.23) (end 74.23 44.23) (width 0.2) (layer "B.Cu") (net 10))
 (segment (start 74.23 44.23) (end 69.39 39.39) (width 0.2) (layer "B.Cu") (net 10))
 (segment (start 84.62975 43.556346) (end 83.956096 44.23) (width 0.2) (layer "B.Cu") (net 10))
 (segment (start 66.26 39.39) (end 47.69 57.96) (width 0.2) (layer "B.Cu") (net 10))
 (segment (start 69.856096 30.38) (end 68.706096 31.53) (width 0.2) (layer "B.Cu") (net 5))
 (segment (start 68.706096 31.53) (end 54.12 31.53) (width 0.2) (layer "B.Cu") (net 5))
 (segment (start 54.12 31.53) (end 47.69 37.96) (width 0.2) (layer "B.Cu") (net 5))
 (segment (start 83.47975 30.38) (end 69.856096 30.38) (width 0.2) (layer "B.Cu") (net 5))
 (segment (start 69.37975 62.87025) (end 68.75 63.5) (width 0.2) (layer "B.Cu") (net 6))
 (segment (start 68.22975 43.08) (end 69.37975 44.23) (width 0.2) (layer "B.Cu") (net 6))
 (segment (start 69.37975 44.23) (end 69.37975 62.87025) (width 0.2) (layer "B.Cu") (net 6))
 (segment (start 68.22975 40.54) (end 70.05 42.36025) (width 0.2) (layer "F.Cu") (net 7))
 (segment (start 70.05 67.2) (end 68.75 68.5) (width 0.2) (layer "F.Cu") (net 7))
 (segment (start 70.05 42.36025) (end 70.05 67.2) (width 0.2) (layer "F.Cu") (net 7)))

